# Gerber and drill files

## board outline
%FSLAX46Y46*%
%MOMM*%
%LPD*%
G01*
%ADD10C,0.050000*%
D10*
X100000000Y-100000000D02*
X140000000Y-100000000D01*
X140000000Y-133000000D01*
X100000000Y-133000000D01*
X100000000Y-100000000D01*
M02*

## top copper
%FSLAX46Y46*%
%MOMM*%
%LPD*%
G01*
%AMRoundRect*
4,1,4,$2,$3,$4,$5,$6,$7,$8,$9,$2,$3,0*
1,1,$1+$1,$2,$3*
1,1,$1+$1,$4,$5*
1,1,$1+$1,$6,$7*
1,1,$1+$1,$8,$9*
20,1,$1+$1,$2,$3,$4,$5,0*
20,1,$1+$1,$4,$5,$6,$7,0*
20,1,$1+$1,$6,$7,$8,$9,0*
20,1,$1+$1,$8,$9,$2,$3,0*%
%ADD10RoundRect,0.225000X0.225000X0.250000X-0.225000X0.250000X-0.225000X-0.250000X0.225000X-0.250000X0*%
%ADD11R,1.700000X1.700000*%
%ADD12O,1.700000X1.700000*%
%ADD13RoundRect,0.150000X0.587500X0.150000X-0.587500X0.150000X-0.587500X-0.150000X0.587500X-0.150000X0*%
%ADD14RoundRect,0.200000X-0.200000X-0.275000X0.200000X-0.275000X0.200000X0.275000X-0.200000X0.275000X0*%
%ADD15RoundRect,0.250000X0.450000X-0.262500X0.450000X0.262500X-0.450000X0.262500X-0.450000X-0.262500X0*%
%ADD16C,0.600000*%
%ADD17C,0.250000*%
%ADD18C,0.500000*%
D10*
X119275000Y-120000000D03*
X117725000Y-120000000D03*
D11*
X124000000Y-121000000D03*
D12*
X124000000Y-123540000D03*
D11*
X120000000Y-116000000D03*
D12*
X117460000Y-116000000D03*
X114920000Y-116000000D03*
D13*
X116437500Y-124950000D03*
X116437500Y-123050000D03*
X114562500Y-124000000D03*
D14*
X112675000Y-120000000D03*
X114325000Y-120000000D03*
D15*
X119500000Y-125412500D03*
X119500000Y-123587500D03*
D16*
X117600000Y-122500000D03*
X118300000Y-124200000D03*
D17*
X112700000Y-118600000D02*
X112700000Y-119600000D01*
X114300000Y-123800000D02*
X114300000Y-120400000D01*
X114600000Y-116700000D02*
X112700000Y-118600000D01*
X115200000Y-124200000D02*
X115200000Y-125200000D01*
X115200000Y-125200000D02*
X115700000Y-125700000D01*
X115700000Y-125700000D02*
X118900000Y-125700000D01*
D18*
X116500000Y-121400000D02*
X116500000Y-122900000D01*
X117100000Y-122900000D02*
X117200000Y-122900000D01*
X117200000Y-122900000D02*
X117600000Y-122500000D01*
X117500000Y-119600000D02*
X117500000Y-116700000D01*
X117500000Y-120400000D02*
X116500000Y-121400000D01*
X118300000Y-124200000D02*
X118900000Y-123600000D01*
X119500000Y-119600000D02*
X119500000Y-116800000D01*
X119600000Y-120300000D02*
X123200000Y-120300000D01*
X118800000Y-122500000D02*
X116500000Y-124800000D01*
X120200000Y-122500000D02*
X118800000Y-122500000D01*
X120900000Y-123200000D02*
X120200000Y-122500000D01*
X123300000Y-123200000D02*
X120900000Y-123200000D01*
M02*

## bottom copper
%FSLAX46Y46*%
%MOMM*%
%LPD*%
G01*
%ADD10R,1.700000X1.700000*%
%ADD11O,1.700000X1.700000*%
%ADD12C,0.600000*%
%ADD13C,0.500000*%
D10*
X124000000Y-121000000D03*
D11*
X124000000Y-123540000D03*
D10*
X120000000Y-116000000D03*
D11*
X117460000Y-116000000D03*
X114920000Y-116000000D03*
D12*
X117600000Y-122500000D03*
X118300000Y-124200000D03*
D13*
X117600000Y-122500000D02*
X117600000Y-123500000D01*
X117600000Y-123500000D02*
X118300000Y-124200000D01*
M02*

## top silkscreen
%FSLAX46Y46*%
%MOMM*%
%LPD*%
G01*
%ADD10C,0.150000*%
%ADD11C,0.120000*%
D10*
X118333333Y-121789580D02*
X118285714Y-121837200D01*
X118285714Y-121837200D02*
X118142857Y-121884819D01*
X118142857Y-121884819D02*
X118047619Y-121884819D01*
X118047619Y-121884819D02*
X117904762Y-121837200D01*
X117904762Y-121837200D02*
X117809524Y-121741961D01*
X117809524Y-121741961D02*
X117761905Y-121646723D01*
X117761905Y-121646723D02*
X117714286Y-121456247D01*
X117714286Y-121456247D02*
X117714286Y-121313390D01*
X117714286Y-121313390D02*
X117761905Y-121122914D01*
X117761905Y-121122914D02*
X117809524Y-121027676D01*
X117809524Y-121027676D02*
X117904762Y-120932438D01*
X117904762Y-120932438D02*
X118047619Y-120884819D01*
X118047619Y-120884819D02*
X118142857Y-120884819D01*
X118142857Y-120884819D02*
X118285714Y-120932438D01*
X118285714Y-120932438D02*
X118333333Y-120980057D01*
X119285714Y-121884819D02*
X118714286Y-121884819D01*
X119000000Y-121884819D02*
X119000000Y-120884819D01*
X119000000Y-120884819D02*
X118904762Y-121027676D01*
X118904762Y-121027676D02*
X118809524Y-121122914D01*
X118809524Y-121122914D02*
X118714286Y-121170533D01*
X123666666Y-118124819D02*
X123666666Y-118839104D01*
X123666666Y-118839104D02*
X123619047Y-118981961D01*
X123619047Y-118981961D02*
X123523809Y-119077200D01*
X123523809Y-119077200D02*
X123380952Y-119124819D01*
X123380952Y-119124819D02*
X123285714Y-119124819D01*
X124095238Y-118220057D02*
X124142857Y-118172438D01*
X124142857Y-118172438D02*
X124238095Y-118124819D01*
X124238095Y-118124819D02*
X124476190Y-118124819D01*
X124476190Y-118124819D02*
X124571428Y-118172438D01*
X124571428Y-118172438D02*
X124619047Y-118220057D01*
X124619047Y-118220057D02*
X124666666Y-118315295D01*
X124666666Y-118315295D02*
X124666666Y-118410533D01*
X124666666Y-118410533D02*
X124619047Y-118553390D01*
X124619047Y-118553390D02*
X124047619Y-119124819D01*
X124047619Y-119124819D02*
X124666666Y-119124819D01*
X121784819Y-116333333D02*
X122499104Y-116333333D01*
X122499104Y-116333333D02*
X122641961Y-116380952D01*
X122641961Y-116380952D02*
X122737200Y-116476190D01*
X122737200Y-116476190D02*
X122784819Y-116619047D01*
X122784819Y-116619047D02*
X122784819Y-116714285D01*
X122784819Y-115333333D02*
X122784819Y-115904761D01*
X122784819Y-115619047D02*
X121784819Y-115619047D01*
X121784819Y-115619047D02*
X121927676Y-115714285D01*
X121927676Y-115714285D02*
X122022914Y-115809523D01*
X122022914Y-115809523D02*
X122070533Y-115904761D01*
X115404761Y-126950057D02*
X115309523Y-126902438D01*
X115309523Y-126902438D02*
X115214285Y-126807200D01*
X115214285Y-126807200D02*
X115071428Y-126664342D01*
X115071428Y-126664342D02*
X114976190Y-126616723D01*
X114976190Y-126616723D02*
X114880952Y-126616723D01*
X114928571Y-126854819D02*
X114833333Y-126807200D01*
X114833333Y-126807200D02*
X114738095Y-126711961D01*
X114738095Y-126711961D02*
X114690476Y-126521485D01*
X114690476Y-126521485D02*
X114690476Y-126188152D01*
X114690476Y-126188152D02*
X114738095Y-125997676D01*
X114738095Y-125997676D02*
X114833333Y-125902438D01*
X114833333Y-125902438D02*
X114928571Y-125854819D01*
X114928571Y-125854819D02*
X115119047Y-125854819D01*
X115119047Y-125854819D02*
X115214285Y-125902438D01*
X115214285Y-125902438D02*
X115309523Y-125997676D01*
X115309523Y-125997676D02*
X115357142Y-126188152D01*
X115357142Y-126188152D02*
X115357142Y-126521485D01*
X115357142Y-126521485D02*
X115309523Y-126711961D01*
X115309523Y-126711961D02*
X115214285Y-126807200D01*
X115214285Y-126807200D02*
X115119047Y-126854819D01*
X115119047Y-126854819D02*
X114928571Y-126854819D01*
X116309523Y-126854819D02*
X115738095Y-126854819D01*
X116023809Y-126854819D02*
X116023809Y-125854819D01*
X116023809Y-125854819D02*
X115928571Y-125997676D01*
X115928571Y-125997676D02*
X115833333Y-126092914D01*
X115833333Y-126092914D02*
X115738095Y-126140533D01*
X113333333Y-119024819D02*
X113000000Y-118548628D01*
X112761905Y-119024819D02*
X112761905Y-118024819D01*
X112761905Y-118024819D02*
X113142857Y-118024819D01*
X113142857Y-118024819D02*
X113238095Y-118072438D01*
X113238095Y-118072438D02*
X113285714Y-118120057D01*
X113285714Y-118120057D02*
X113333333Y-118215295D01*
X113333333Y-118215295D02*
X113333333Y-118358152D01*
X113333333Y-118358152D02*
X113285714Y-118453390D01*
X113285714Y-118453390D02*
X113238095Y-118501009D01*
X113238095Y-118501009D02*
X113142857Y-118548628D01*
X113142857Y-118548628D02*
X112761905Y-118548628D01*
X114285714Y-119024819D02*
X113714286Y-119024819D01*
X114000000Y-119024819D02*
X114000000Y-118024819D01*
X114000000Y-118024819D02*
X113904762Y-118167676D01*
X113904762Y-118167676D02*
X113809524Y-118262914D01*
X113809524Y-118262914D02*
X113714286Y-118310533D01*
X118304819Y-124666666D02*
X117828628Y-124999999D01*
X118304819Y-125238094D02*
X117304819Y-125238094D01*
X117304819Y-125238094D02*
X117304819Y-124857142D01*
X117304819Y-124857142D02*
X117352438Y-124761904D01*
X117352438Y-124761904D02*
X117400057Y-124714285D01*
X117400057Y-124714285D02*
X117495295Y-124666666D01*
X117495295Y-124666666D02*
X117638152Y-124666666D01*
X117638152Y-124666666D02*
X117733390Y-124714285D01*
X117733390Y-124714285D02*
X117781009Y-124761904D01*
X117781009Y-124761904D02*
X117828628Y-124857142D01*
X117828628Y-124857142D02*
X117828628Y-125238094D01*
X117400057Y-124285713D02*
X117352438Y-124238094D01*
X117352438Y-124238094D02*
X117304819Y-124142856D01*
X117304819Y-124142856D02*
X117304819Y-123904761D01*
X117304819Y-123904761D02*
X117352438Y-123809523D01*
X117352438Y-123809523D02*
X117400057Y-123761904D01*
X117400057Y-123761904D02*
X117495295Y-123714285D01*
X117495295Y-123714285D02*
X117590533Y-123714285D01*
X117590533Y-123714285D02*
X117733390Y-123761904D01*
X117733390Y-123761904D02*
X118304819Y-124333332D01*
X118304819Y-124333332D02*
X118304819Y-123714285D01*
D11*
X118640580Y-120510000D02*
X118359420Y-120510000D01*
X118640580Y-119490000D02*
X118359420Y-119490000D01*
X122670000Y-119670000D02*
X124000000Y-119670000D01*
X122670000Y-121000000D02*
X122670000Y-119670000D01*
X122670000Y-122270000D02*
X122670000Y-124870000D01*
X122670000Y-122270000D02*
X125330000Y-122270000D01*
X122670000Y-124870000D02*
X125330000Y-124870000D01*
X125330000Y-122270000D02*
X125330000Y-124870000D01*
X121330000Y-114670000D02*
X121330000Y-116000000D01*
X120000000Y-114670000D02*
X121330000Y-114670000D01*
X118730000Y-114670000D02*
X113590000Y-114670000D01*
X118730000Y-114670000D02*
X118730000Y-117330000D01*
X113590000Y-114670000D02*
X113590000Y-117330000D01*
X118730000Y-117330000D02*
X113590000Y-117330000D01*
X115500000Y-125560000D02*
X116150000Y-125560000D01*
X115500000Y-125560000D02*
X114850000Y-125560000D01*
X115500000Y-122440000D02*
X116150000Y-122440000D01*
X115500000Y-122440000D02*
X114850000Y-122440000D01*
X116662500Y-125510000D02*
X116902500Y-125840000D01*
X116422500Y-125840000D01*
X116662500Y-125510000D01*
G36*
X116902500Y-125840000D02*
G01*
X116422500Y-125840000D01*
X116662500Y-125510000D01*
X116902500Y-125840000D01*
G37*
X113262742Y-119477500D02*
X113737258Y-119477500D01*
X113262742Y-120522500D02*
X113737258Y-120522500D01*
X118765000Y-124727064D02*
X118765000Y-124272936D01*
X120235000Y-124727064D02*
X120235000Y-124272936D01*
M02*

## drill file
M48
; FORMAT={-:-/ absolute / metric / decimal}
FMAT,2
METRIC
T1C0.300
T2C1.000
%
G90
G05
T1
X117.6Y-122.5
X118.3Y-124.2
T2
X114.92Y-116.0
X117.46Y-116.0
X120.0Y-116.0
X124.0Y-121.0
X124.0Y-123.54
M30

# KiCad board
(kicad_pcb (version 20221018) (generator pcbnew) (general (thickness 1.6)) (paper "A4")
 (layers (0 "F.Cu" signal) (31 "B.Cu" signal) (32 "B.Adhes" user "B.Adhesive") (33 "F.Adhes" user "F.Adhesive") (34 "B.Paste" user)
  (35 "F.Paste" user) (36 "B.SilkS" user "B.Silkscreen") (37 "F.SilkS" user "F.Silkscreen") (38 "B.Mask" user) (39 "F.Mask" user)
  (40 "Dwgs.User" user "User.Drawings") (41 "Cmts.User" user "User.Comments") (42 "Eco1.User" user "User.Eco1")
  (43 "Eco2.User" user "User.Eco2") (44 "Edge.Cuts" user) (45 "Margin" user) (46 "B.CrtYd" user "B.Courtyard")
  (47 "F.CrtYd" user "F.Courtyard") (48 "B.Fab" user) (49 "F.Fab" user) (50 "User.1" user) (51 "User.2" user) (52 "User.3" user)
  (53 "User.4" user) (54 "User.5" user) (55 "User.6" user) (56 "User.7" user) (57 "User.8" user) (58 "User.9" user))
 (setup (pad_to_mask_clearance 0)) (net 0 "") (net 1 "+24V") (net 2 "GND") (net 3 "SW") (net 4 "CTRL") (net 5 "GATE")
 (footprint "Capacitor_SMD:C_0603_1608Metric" (layer "F.Cu") (at 118.5 120 180)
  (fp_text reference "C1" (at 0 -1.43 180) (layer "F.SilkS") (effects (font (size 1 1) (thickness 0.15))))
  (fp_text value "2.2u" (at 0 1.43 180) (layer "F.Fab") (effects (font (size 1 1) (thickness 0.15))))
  (fp_line (start -0.14058 -0.51) (end 0.14058 -0.51) (stroke (width 0.12) (type solid)) (layer "F.SilkS"))
  (fp_line (start -0.14058 0.51) (end 0.14058 0.51) (stroke (width 0.12) (type solid)) (layer "F.SilkS"))
  (pad "1" smd roundrect (at -0.775 0 180) (size 0.9 0.95) (layers "F.Cu" "F.Paste" "F.Mask") (roundrect_rratio 0.25) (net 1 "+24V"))
  (pad "2" smd roundrect (at 0.775 0 180) (size 0.9 0.95) (layers "F.Cu" "F.Paste" "F.Mask") (roundrect_rratio 0.25) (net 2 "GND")))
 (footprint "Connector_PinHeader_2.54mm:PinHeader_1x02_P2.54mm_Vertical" (layer "F.Cu") (at 124 121)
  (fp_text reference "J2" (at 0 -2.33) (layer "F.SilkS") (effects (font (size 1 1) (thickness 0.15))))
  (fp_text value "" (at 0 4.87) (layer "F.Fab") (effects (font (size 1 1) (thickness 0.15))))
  (fp_line (start -1.33 -1.33) (end 0 -1.33) (stroke (width 0.12) (type solid)) (layer "F.SilkS"))
  (fp_line (start -1.33 0) (end -1.33 -1.33) (stroke (width 0.12) (type solid)) (layer "F.SilkS"))
  (fp_line (start -1.33 1.27) (end -1.33 3.87) (stroke (width 0.12) (type solid)) (layer "F.SilkS"))
  (fp_line (start -1.33 1.27) (end 1.33 1.27) (stroke (width 0.12) (type solid)) (layer "F.SilkS"))
  (fp_line (start -1.33 3.87) (end 1.33 3.87) (stroke (width 0.12) (type solid)) (layer "F.SilkS"))
  (fp_line (start 1.33 1.27) (end 1.33 3.87) (stroke (width 0.12) (type solid)) (layer "F.SilkS"))
  (pad "1" thru_hole rect (at 0 0) (size 1.7 1.7) (drill 1) (layers "*.Cu" "*.Mask") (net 1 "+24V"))
  (pad "2" thru_hole oval (at 0 2.54) (size 1.7 1.7) (drill 1) (layers "*.Cu" "*.Mask") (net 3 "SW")))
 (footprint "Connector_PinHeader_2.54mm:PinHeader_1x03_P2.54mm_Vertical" (layer "F.Cu") (at 120 116 -90)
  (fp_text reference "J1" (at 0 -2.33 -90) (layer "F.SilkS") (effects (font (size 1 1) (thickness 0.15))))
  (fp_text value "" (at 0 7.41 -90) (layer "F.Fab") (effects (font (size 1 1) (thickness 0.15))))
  (fp_line (start -1.33 -1.33) (end 0 -1.33) (stroke (width 0.12) (type solid)) (layer "F.SilkS"))
  (fp_line (start -1.33 0) (end -1.33 -1.33) (stroke (width 0.12) (type solid)) (layer "F.SilkS"))
  (fp_line (start -1.33 1.27) (end -1.33 6.41) (stroke (width 0.12) (type solid)) (layer "F.SilkS"))
  (fp_line (start -1.33 1.27) (end 1.33 1.27) (stroke (width 0.12) (type solid)) (layer "F.SilkS"))
  (fp_line (start -1.33 6.41) (end 1.33 6.41) (stroke (width 0.12) (type solid)) (layer "F.SilkS"))
  (fp_line (start 1.33 1.27) (end 1.33 6.41) (stroke (width 0.12) (type solid)) (layer "F.SilkS"))
  (pad "1" thru_hole rect (at 0 0 270) (size 1.7 1.7) (drill 1) (layers "*.Cu" "*.Mask") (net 1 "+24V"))
  (pad "2" thru_hole oval (at 0 2.54 270) (size 1.7 1.7) (drill 1) (layers "*.Cu" "*.Mask") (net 2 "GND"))
  (pad "3" thru_hole oval (at 0 5.08 270) (size 1.7 1.7) (drill 1) (layers "*.Cu" "*.Mask") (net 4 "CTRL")))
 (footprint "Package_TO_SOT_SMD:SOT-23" (layer "F.Cu") (at 115.5 124 180)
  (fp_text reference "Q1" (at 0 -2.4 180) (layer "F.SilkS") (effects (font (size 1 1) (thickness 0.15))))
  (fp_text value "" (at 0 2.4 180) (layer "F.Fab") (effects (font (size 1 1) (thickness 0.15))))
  (fp_line (start 0 -1.56) (end -0.65 -1.56) (stroke (width 0.12) (type solid)) (layer "F.SilkS"))
  (fp_line (start 0 -1.56) (end 0.65 -1.56) (stroke (width 0.12) (type solid)) (layer "F.SilkS"))
  (fp_line (start 0 1.56) (end -0.65 1.56) (stroke (width 0.12) (type solid)) (layer "F.SilkS"))
  (fp_line (start 0 1.56) (end 0.65 1.56) (stroke (width 0.12) (type solid)) (layer "F.SilkS"))
  (fp_poly
   (pts (xy -1.1625 -1.51) (xy -1.4025 -1.84) (xy -0.9225 -1.84) (xy -1.1625 -1.51)) (stroke (width 0.12) (type solid)) (fill solid)
   (layer "F.SilkS"))
  (pad "1" smd roundrect (at -0.9375 -0.95 180) (size 1.475 0.6) (layers "F.Cu" "F.Paste" "F.Mask") (roundrect_rratio 0.25) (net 3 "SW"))
  (pad "2" smd roundrect (at -0.9375 0.95 180) (size 1.475 0.6) (layers "F.Cu" "F.Paste" "F.Mask") (roundrect_rratio 0.25) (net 2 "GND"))
  (pad "3" smd roundrect (at 0.9375 0 180) (size 1.475 0.6) (layers "F.Cu" "F.Paste" "F.Mask") (roundrect_rratio 0.25) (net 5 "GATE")))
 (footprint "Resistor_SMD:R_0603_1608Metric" (layer "F.Cu") (at 113.5 120)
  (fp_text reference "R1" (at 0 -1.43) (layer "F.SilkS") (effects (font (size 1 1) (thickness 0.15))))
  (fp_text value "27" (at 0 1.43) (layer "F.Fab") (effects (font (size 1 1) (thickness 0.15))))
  (fp_line (start -0.237258 -0.5225) (end 0.237258 -0.5225) (stroke (width 0.12) (type solid)) (layer "F.SilkS"))
  (fp_line (start -0.237258 0.5225) (end 0.237258 0.5225) (stroke (width 0.12) (type solid)) (layer "F.SilkS"))
  (pad "1" smd roundrect (at -0.825 0) (size 0.8 0.95) (layers "F.Cu" "F.Paste" "F.Mask") (roundrect_rratio 0.25) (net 4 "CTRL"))
  (pad "2" smd roundrect (at 0.825 0) (size 0.8 0.95) (layers "F.Cu" "F.Paste" "F.Mask") (roundrect_rratio 0.25) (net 5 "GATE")))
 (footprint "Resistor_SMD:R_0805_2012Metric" (layer "F.Cu") (at 119.5 124.5 90)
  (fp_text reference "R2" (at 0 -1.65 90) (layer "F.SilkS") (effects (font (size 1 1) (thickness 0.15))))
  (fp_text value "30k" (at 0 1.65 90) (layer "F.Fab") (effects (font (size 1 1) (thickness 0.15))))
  (fp_line (start -0.227064 -0.735) (end 0.227064 -0.735) (stroke (width 0.12) (type solid)) (layer "F.SilkS"))
  (fp_line (start -0.227064 0.735) (end 0.227064 0.735) (stroke (width 0.12) (type solid)) (layer "F.SilkS"))
  (pad "1" smd roundrect (at -0.9125 0 90) (size 1.025 1.4) (layers "F.Cu" "F.Paste" "F.Mask") (roundrect_rratio 0.243902) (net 5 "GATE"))
  (pad "2" smd roundrect (at 0.9125 0 90) (size 1.025 1.4) (layers "F.Cu" "F.Paste" "F.Mask") (roundrect_rratio 0.243902) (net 2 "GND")))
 (gr_rect (start 100 100) (end 140 133) (stroke (width 0.05) (type default)) (fill none) (layer "Edge.Cuts"))
 (segment (start 112.7 118.6) (end 112.7 119.6) (width 0.25) (layer "F.Cu") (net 4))
 (segment (start 114.3 123.8) (end 114.3 120.4) (width 0.25) (layer "F.Cu") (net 5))
 (segment (start 114.6 116.7) (end 112.7 118.6) (width 0.25) (layer "F.Cu") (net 4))
 (segment (start 115.2 124.2) (end 115.2 125.2) (width 0.25) (layer "F.Cu") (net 5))
 (segment (start 115.2 125.2) (end 115.7 125.7) (width 0.25) (layer "F.Cu") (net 5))
 (segment (start 115.7 125.7) (end 118.9 125.7) (width 0.25) (layer "F.Cu") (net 5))
 (segment (start 116.5 121.4) (end 116.5 122.9) (width 0.5) (layer "F.Cu") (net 2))
 (segment (start 117.1 122.9) (end 117.2 122.9) (width 0.5) (layer "F.Cu") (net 2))
 (segment (start 117.2 122.9) (end 117.6 122.5) (width 0.5) (layer "F.Cu") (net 2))
 (segment (start 117.5 119.6) (end 117.5 116.7) (width 0.5) (layer "F.Cu") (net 2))
 (segment (start 117.5 120.4) (end 116.5 121.4) (width 0.5) (layer "F.Cu") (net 2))
 (segment (start 118.3 124.2) (end 118.9 123.6) (width 0.5) (layer "F.Cu") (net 2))
 (segment (start 119.5 119.6) (end 119.5 116.8) (width 0.5) (layer "F.Cu") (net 1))
 (segment (start 119.6 120.3) (end 123.2 120.3) (width 0.5) (layer "F.Cu") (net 1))
 (via (at 117.6 122.5) (size 0.6) (drill 0.3) (layers "F.Cu" "B.Cu") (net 2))
 (via (at 118.3 124.2) (size 0.6) (drill 0.3) (layers "F.Cu" "B.Cu") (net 2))
 (segment (start 117.6 122.5) (end 117.6 123.5) (width 0.5) (layer "B.Cu") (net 2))
 (segment (start 117.6 123.5) (end 118.3 124.2) (width 0.5) (layer "B.Cu") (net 2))
 (segment (start 118.8 122.5) (end 116.5 124.8) (width 0.5) (layer "F.Cu") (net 3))
 (segment (start 120.2 122.5) (end 118.8 122.5) (width 0.5) (layer "F.Cu") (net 3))
 (segment (start 120.9 123.2) (end 120.2 122.5) (width 0.5) (layer "F.Cu") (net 3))
 (segment (start 123.3 123.2) (end 120.9 123.2) (width 0.5) (layer "F.Cu") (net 3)))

